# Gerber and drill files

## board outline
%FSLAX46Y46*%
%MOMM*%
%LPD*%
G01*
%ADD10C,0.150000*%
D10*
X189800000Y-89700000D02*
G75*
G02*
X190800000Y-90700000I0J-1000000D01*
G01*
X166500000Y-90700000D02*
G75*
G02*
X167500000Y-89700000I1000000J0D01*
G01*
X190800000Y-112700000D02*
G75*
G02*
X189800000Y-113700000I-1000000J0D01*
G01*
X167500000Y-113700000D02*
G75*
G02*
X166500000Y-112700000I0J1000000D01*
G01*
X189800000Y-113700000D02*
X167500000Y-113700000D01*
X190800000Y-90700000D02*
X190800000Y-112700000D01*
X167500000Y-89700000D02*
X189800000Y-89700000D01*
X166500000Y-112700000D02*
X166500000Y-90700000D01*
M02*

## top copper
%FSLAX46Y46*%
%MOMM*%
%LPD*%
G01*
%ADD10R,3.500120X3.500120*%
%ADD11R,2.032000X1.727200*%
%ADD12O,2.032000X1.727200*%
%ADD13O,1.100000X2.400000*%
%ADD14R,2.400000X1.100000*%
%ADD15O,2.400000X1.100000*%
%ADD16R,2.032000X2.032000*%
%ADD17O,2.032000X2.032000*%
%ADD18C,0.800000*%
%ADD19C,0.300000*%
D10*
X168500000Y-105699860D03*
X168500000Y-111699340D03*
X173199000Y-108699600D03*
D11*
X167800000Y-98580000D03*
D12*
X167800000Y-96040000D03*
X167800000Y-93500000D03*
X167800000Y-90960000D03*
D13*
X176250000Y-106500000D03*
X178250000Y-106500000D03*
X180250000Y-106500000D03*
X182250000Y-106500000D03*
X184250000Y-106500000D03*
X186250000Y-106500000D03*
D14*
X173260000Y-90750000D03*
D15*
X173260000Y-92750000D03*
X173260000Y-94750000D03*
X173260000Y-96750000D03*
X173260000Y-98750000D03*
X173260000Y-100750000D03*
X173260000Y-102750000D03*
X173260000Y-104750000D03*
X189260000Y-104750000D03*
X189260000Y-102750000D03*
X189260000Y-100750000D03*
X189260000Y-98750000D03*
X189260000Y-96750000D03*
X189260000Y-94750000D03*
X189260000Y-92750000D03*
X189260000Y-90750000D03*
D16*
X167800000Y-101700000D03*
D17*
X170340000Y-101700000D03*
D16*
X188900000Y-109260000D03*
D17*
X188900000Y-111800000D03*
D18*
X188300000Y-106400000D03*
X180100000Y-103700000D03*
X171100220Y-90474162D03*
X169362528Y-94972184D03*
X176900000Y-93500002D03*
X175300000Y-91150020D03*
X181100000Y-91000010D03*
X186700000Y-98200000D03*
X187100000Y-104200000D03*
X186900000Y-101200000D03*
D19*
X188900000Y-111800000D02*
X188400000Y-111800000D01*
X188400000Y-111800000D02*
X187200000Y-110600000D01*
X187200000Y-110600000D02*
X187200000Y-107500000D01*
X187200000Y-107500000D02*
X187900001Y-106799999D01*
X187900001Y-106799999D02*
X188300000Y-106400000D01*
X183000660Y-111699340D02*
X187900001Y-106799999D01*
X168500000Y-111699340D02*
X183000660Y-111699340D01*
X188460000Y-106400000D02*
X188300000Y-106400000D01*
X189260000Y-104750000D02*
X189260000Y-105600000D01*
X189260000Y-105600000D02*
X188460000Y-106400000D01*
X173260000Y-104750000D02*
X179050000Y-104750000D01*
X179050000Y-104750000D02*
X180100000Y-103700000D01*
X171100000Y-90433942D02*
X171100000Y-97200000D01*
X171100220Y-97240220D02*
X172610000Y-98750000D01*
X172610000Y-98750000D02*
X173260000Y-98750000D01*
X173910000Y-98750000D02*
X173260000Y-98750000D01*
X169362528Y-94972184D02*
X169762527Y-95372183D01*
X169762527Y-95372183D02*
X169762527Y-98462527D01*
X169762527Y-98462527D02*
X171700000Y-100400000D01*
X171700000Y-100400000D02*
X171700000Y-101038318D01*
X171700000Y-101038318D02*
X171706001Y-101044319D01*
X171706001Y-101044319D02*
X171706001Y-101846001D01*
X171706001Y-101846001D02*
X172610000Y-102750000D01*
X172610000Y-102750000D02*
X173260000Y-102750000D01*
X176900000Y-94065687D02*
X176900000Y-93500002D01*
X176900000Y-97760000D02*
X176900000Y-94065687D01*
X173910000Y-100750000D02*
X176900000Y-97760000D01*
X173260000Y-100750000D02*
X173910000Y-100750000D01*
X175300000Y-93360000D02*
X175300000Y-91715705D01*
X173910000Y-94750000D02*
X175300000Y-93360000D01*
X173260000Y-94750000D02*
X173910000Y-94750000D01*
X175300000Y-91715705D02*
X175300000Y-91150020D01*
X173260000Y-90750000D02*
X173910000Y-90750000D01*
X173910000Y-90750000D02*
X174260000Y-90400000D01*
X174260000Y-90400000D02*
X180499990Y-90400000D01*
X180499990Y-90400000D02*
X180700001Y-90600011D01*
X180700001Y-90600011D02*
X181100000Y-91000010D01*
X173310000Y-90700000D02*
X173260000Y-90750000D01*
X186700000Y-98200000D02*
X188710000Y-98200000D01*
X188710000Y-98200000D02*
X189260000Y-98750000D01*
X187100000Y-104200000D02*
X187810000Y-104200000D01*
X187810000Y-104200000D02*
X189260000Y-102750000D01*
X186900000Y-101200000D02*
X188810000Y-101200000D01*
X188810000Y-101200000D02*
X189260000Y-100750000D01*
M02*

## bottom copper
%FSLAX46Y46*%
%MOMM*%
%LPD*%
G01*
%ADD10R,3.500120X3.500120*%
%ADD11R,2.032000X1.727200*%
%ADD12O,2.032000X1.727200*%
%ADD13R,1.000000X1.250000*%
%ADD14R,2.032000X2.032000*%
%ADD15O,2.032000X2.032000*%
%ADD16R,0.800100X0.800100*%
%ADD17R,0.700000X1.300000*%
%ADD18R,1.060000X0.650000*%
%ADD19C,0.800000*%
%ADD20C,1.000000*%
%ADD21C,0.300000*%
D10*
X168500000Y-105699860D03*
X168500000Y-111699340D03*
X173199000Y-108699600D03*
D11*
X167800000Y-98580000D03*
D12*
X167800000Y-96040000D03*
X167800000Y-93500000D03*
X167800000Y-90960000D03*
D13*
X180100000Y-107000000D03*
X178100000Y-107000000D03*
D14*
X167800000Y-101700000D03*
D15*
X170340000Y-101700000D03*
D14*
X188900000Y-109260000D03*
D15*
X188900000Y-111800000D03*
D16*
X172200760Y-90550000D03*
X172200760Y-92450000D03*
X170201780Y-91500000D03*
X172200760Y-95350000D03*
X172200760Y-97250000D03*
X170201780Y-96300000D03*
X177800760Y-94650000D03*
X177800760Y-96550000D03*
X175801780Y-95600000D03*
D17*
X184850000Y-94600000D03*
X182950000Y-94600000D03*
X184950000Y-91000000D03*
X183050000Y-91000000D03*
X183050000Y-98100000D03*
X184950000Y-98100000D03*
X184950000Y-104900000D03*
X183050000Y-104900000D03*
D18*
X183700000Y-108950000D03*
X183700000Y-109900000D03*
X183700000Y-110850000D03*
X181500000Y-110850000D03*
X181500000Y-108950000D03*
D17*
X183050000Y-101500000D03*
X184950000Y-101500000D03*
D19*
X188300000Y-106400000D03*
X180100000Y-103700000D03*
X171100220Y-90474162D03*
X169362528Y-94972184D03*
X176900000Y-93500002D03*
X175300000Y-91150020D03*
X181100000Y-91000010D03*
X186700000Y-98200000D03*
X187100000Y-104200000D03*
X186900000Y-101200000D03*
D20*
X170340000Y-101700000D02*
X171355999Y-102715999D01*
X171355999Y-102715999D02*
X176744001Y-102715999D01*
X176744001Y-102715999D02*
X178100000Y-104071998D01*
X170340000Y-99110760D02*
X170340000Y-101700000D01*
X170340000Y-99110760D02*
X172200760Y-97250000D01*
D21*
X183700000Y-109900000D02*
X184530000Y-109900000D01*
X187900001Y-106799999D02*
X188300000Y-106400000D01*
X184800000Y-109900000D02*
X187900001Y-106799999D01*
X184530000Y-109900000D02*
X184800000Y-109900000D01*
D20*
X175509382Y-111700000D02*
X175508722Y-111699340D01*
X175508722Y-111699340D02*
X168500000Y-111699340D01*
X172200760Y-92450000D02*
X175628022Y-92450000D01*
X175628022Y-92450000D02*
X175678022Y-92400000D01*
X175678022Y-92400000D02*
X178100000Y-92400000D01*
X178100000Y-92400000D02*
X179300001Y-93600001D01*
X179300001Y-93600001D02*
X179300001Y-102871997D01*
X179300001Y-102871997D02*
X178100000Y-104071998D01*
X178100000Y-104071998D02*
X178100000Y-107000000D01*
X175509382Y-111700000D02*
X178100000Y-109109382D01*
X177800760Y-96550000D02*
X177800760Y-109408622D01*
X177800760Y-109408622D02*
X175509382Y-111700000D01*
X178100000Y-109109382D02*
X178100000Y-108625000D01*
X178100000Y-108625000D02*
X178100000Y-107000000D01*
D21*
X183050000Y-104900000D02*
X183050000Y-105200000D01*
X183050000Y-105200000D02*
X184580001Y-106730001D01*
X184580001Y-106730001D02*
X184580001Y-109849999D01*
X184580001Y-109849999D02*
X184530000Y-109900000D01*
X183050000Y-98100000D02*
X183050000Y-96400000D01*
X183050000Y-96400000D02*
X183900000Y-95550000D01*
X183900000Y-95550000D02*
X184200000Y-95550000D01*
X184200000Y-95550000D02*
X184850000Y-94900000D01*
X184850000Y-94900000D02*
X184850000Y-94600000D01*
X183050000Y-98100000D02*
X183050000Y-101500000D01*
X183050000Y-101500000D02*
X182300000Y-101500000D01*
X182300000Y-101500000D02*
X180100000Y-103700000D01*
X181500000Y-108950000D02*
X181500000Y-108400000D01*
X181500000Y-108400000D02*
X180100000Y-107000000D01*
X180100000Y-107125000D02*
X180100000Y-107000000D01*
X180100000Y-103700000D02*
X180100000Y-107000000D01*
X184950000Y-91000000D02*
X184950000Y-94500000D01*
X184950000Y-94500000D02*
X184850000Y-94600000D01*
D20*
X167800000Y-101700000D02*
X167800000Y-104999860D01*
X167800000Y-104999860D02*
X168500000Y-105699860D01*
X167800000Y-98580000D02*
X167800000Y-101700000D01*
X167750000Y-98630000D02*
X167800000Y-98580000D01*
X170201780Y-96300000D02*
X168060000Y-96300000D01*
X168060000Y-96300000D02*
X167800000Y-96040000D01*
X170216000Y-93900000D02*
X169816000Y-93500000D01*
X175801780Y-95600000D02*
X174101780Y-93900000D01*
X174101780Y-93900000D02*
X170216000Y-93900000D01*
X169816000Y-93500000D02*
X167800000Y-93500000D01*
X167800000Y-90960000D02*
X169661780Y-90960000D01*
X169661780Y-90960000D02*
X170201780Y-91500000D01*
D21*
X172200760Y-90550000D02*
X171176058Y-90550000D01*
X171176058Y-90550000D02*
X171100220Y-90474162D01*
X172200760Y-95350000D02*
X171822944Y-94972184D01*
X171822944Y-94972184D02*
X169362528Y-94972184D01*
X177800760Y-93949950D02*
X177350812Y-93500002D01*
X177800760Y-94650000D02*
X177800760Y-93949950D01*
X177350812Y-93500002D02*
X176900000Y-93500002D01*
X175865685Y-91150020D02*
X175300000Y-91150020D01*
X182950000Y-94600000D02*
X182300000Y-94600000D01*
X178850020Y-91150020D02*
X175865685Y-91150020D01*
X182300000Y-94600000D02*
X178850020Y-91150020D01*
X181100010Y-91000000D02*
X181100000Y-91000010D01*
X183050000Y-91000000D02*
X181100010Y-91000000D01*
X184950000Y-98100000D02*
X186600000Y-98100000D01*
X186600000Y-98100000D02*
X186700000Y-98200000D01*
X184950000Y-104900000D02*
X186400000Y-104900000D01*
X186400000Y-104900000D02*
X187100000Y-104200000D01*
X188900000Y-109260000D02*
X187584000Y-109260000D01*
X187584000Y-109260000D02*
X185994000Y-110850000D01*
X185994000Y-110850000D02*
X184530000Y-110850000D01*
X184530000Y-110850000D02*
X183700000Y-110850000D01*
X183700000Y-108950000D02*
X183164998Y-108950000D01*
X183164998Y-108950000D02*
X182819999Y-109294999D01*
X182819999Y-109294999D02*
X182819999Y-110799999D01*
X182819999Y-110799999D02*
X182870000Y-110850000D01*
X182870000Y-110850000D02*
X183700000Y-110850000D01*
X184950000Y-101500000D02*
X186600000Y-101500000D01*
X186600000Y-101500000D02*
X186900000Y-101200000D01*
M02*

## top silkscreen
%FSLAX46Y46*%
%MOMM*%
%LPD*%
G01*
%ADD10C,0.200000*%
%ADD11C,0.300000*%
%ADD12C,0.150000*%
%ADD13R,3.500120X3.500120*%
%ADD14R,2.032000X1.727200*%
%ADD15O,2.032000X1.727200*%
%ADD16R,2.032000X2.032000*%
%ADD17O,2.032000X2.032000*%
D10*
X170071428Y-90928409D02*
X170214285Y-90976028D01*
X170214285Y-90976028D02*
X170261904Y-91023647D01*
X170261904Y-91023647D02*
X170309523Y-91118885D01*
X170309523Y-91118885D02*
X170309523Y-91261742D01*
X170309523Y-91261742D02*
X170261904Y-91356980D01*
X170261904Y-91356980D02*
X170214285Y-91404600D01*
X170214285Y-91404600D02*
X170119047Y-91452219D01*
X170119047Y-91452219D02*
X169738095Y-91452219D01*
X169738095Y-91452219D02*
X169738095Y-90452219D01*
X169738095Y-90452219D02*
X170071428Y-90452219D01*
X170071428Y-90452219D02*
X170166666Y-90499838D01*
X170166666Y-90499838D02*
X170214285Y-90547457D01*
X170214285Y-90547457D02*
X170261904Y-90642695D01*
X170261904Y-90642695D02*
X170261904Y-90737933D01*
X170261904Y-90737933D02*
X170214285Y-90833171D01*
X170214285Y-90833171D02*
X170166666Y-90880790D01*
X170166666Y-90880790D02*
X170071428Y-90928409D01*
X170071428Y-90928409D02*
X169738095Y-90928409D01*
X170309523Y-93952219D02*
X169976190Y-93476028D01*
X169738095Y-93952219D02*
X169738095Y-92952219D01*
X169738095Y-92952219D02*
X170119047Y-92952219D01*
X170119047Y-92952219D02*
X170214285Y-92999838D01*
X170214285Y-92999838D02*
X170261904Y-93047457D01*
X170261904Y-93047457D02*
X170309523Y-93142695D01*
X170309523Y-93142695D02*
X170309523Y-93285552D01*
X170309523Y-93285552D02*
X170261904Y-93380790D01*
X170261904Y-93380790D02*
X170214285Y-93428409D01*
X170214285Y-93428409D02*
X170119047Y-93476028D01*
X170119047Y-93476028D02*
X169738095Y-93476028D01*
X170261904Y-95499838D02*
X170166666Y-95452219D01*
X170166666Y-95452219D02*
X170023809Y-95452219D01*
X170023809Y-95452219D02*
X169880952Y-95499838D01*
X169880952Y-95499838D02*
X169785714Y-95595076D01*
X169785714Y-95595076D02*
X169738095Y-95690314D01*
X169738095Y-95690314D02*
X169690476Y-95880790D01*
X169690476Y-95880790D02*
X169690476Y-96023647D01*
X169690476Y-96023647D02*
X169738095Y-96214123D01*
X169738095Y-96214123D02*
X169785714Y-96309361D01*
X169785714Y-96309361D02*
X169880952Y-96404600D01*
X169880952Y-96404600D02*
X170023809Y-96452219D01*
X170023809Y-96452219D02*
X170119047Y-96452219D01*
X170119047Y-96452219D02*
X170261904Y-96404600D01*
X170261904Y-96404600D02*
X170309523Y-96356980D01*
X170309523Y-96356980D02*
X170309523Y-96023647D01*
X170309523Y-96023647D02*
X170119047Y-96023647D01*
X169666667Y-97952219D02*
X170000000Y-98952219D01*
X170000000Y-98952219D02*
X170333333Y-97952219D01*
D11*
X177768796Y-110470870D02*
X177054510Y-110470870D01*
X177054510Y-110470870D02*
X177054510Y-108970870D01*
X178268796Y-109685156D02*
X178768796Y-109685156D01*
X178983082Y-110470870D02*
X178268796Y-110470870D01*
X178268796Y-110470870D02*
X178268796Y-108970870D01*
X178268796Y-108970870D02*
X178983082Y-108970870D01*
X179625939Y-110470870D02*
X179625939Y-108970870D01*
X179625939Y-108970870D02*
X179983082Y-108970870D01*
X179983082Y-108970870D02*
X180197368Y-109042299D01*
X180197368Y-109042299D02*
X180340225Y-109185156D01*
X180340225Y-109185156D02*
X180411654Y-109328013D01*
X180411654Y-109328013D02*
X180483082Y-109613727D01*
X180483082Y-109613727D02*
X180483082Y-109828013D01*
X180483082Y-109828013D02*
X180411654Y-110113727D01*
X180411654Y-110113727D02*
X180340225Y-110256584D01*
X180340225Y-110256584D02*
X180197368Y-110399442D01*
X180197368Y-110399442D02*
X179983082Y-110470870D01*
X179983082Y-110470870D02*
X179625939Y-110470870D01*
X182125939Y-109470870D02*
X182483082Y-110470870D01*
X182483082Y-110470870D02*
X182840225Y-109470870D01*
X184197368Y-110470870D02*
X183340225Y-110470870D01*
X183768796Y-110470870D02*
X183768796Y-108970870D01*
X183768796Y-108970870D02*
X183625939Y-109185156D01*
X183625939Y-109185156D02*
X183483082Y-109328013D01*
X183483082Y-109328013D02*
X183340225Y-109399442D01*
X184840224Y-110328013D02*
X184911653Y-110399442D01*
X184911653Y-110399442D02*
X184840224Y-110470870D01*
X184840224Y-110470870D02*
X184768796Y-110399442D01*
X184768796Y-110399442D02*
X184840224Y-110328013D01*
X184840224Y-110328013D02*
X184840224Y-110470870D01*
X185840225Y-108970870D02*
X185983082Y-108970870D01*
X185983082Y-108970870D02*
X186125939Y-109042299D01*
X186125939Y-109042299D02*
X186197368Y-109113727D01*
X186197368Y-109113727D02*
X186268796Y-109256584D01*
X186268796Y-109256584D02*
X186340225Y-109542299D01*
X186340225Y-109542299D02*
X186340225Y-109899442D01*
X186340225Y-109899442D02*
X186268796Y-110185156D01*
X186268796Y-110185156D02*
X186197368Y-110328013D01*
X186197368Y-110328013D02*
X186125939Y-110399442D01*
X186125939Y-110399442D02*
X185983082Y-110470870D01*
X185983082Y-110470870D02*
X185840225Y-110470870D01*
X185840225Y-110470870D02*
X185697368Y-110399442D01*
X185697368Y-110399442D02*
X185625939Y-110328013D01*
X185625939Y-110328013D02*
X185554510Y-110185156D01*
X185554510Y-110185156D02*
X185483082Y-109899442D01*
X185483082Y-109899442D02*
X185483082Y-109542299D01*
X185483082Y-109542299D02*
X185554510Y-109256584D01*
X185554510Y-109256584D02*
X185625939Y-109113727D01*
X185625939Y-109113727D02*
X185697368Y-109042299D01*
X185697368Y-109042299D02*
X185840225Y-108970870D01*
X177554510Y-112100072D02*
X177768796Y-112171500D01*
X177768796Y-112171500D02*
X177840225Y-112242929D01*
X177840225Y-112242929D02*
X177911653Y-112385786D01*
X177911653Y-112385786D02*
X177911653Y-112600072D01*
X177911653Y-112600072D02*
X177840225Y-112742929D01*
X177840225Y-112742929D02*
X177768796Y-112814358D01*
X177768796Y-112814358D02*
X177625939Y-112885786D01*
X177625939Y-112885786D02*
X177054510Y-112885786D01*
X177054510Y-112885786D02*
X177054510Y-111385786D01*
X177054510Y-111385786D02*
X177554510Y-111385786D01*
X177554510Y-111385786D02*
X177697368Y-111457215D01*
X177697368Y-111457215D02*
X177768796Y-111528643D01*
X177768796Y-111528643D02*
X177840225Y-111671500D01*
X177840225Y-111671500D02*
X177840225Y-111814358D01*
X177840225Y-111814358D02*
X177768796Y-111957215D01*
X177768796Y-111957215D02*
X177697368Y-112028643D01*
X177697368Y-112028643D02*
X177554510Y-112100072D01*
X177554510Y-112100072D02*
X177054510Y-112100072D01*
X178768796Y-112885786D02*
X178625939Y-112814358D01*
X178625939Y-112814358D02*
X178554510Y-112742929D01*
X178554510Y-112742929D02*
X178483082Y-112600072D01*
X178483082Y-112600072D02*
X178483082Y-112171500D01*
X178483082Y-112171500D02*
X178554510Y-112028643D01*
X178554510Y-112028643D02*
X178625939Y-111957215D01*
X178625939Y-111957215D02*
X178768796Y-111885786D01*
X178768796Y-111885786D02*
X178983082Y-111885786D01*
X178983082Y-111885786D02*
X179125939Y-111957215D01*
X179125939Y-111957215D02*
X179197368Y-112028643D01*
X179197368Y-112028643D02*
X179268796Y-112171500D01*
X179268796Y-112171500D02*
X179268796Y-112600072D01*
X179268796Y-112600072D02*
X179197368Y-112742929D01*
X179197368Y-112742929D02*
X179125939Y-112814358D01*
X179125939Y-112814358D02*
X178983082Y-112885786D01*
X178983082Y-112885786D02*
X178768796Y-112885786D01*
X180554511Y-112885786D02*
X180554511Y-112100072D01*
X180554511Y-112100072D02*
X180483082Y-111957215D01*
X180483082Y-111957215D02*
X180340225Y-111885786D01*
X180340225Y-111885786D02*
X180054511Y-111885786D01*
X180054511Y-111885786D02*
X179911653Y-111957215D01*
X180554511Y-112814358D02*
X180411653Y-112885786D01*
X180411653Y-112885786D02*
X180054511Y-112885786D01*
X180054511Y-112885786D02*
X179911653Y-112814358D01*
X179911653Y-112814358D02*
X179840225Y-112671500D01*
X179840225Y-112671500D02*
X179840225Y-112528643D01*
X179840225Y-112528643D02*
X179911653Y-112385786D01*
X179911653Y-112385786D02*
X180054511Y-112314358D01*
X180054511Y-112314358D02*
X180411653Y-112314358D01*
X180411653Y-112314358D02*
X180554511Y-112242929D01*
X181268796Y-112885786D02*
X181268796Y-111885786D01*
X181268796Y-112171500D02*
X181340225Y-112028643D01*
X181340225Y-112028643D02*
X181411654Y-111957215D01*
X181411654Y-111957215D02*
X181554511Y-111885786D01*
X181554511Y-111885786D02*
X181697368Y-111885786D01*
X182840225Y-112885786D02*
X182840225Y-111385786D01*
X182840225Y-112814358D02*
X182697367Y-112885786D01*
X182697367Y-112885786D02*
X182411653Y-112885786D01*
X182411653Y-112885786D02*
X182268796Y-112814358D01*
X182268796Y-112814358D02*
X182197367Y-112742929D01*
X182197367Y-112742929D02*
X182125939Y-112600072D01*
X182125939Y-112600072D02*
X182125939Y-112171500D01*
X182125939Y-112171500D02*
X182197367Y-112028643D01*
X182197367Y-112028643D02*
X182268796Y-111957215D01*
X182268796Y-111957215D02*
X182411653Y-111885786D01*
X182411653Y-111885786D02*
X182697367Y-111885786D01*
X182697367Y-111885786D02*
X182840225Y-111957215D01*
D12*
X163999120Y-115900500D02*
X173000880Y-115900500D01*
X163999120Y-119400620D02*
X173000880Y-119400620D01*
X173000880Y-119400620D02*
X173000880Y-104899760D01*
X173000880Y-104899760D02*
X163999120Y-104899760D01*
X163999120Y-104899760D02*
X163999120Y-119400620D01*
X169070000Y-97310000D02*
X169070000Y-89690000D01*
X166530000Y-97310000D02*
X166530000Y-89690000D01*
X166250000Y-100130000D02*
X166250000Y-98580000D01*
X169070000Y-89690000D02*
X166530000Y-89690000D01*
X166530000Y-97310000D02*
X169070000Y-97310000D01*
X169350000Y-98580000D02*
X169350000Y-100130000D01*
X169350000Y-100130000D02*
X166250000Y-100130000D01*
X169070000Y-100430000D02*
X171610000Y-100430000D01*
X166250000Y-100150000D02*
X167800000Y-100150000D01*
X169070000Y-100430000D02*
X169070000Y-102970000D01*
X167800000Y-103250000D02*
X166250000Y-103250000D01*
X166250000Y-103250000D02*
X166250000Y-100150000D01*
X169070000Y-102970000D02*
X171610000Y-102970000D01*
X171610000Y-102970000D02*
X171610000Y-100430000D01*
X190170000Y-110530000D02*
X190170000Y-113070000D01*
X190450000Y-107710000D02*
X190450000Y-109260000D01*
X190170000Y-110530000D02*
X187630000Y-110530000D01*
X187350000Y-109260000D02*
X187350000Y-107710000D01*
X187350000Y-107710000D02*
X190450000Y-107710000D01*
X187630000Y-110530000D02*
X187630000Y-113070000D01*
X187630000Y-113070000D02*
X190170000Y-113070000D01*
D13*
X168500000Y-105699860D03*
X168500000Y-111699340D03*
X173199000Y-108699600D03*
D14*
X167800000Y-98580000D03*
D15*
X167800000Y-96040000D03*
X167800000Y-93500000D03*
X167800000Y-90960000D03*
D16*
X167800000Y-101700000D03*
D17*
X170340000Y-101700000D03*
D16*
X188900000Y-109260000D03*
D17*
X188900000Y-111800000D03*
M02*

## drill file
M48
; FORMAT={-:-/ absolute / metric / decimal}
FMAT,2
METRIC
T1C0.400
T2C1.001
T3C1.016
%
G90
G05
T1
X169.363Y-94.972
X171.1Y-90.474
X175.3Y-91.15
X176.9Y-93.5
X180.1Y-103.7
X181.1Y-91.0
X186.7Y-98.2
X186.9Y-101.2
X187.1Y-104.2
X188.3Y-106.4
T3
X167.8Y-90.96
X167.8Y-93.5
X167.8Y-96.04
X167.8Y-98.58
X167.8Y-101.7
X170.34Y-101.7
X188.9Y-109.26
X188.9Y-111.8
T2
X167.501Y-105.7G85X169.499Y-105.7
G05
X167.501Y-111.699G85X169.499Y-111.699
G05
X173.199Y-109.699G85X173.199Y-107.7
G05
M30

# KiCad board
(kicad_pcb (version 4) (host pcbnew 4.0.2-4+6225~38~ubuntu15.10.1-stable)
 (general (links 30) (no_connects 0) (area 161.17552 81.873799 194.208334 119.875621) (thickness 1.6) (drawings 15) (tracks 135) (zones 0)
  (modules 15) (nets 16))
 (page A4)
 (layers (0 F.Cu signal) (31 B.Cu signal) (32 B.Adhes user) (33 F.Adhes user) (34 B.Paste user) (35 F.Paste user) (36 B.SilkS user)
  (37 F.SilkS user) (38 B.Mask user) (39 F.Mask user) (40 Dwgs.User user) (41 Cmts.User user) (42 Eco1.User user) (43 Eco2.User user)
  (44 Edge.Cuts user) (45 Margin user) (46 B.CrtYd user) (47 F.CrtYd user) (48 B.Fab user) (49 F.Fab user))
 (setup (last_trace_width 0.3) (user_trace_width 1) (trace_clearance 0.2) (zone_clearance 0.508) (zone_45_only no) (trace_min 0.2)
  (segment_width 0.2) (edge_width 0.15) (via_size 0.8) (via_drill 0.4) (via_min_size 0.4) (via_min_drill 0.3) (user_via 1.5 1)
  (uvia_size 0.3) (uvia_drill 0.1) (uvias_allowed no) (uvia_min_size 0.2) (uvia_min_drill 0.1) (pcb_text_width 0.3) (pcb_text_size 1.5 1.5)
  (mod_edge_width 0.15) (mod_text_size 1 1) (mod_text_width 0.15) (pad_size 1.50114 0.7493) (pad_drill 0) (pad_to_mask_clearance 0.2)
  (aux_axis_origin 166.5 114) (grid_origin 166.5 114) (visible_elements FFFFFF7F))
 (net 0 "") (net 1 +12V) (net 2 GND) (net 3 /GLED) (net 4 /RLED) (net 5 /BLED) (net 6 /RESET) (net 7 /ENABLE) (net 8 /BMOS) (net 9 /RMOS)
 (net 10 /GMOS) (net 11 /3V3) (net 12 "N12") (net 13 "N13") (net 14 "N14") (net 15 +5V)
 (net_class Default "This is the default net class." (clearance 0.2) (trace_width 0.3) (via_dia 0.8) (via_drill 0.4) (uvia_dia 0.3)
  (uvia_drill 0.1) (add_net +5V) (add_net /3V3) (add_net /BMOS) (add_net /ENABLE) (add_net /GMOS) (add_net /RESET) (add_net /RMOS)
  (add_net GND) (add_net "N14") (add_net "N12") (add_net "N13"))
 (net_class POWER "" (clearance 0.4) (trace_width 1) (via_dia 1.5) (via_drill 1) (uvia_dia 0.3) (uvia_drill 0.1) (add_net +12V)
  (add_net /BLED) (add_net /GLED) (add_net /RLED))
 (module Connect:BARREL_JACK (layer F.Cu) (at 168.5 111.9 90)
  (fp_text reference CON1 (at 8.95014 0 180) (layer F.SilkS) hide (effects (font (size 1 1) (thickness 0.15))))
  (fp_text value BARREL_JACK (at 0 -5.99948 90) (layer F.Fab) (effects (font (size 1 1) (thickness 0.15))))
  (fp_line (start -4.0005 -4.50088) (end -4.0005 4.50088) (layer F.SilkS) (width 0.15))
  (fp_line (start -7.50062 -4.50088) (end -7.50062 4.50088) (layer F.SilkS) (width 0.15))
  (fp_line (start -7.50062 4.50088) (end 7.00024 4.50088) (layer F.SilkS) (width 0.15))
  (fp_line (start 7.00024 4.50088) (end 7.00024 -4.50088) (layer F.SilkS) (width 0.15))
  (fp_line (start 7.00024 -4.50088) (end -7.50062 -4.50088) (layer F.SilkS) (width 0.15))
  (pad 1 thru_hole rect (at 6.20014 0 90) (size 3.50012 3.50012) (drill oval 1.00076 2.99974) (layers *.Cu *.Mask F.SilkS) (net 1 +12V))
  (pad 2 thru_hole rect (at 0.20066 0 90) (size 3.50012 3.50012) (drill oval 1.00076 2.99974) (layers *.Cu *.Mask F.SilkS) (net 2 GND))
  (pad 3 thru_hole rect (at 3.2004 4.699 90) (size 3.50012 3.50012) (drill oval 2.99974 1.00076) (layers *.Cu *.Mask F.SilkS)))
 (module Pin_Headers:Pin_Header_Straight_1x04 (layer F.Cu) (at 167.8 98.58 180)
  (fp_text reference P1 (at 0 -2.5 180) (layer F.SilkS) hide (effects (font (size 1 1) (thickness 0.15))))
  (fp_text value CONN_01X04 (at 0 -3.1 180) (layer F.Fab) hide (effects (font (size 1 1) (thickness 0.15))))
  (fp_line (start -1.27 1.27) (end -1.27 8.89) (layer F.SilkS) (width 0.15))
  (fp_line (start 1.27 1.27) (end 1.27 8.89) (layer F.SilkS) (width 0.15))
  (fp_line (start 1.55 -1.55) (end 1.55 0) (layer F.SilkS) (width 0.15))
  (fp_line (start -1.27 8.89) (end 1.27 8.89) (layer F.SilkS) (width 0.15))
  (fp_line (start 1.27 1.27) (end -1.27 1.27) (layer F.SilkS) (width 0.15))
  (fp_line (start -1.55 0) (end -1.55 -1.55) (layer F.SilkS) (width 0.15))
  (fp_line (start -1.55 -1.55) (end 1.55 -1.55) (layer F.SilkS) (width 0.15))
  (pad 1 thru_hole rect (at 0 0 180) (size 2.032 1.7272) (drill 1.016) (layers *.Cu *.Mask F.SilkS) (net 1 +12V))
  (pad 2 thru_hole oval (at 0 2.54 180) (size 2.032 1.7272) (drill 1.016) (layers *.Cu *.Mask F.SilkS) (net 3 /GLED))
  (pad 3 thru_hole oval (at 0 5.08 180) (size 2.032 1.7272) (drill 1.016) (layers *.Cu *.Mask F.SilkS) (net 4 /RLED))
  (pad 4 thru_hole oval (at 0 7.62 180) (size 2.032 1.7272) (drill 1.016) (layers *.Cu *.Mask F.SilkS) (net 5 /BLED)))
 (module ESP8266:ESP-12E (layer F.Cu) (at 173.26 90.75)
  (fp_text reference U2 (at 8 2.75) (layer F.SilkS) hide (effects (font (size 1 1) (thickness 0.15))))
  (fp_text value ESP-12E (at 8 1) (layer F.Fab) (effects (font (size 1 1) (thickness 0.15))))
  (pad 9 smd oval (at 2.99 15.75 90) (size 2.4 1.1) (layers F.Cu F.Paste F.Mask))
  (pad 10 smd oval (at 4.99 15.75 90) (size 2.4 1.1) (layers F.Cu F.Paste F.Mask))
  (pad 11 smd oval (at 6.99 15.75 90) (size 2.4 1.1) (layers F.Cu F.Paste F.Mask))
  (pad 12 smd oval (at 8.99 15.75 90) (size 2.4 1.1) (layers F.Cu F.Paste F.Mask))
  (pad 13 smd oval (at 10.99 15.75 90) (size 2.4 1.1) (layers F.Cu F.Paste F.Mask))
  (pad 14 smd oval (at 12.99 15.75 90) (size 2.4 1.1) (layers F.Cu F.Paste F.Mask))
  (pad 1 smd rect (at 0 0) (size 2.4 1.1) (layers F.Cu F.Paste F.Mask) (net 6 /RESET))
  (pad 2 smd oval (at 0 2) (size 2.4 1.1) (layers F.Cu F.Paste F.Mask))
  (pad 3 smd oval (at 0 4) (size 2.4 1.1) (layers F.Cu F.Paste F.Mask) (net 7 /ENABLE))
  (pad 4 smd oval (at 0 6) (size 2.4 1.1) (layers F.Cu F.Paste F.Mask))
  (pad 5 smd oval (at 0 8) (size 2.4 1.1) (layers F.Cu F.Paste F.Mask) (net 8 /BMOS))
  (pad 6 smd oval (at 0 10) (size 2.4 1.1) (layers F.Cu F.Paste F.Mask) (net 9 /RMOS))
  (pad 7 smd oval (at 0 12) (size 2.4 1.1) (layers F.Cu F.Paste F.Mask) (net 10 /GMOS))
  (pad 8 smd oval (at 0 14) (size 2.4 1.1) (layers F.Cu F.Paste F.Mask) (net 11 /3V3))
  (pad 15 smd oval (at 16 14) (size 2.4 1.1) (layers F.Cu F.Paste F.Mask) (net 2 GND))
  (pad 16 smd oval (at 16 12) (size 2.4 1.1) (layers F.Cu F.Paste F.Mask) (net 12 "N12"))
  (pad 17 smd oval (at 16 10) (size 2.4 1.1) (layers F.Cu F.Paste F.Mask) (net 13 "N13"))
  (pad 18 smd oval (at 16 8) (size 2.4 1.1) (layers F.Cu F.Paste F.Mask) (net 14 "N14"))
  (pad 19 smd oval (at 16 6) (size 2.4 1.1) (layers F.Cu F.Paste F.Mask))
  (pad 20 smd oval (at 16 4) (size 2.4 1.1) (layers F.Cu F.Paste F.Mask))
  (pad 21 smd oval (at 16 2) (size 2.4 1.1) (layers F.Cu F.Paste F.Mask))
  (pad 22 smd oval (at 16 0) (size 2.4 1.1) (layers F.Cu F.Paste F.Mask)))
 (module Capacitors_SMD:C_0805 (layer B.Cu) (at 179.1 107 180)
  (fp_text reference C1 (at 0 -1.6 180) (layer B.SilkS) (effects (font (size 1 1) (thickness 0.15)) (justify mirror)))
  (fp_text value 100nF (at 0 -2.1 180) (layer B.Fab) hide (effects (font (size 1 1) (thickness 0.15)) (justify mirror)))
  (pad 1 smd rect (at -1 0 180) (size 1 1.25) (layers B.Cu B.Paste B.Mask) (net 11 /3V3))
  (pad 2 smd rect (at 1 0 180) (size 1 1.25) (layers B.Cu B.Paste B.Mask) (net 2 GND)))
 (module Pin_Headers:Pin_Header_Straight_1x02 (layer F.Cu) (at 167.8 101.7 90)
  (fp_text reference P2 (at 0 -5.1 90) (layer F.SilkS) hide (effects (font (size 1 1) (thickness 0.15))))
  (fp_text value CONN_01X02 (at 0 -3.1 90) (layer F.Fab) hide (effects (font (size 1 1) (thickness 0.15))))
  (fp_line (start 1.27 1.27) (end 1.27 3.81) (layer F.SilkS) (width 0.15))
  (fp_line (start 1.55 -1.55) (end 1.55 0) (layer F.SilkS) (width 0.15))
  (fp_line (start 1.27 1.27) (end -1.27 1.27) (layer F.SilkS) (width 0.15))
  (fp_line (start -1.55 0) (end -1.55 -1.55) (layer F.SilkS) (width 0.15))
  (fp_line (start -1.55 -1.55) (end 1.55 -1.55) (layer F.SilkS) (width 0.15))
  (fp_line (start -1.27 1.27) (end -1.27 3.81) (layer F.SilkS) (width 0.15))
  (fp_line (start -1.27 3.81) (end 1.27 3.81) (layer F.SilkS) (width 0.15))
  (pad 1 thru_hole rect (at 0 0 90) (size 2.032 2.032) (drill 1.016) (layers *.Cu *.Mask F.SilkS) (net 1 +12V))
  (pad 2 thru_hole oval (at 0 2.54 90) (size 2.032 2.032) (drill 1.016) (layers *.Cu *.Mask F.SilkS) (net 2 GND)))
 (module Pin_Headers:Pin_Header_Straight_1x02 (layer F.Cu) (at 188.9 109.26)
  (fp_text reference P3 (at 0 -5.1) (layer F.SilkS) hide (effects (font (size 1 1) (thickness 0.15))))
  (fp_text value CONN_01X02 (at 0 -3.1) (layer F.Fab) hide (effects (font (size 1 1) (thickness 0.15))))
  (fp_line (start 1.27 1.27) (end 1.27 3.81) (layer F.SilkS) (width 0.15))
  (fp_line (start 1.55 -1.55) (end 1.55 0) (layer F.SilkS) (width 0.15))
  (fp_line (start 1.27 1.27) (end -1.27 1.27) (layer F.SilkS) (width 0.15))
  (fp_line (start -1.55 0) (end -1.55 -1.55) (layer F.SilkS) (width 0.15))
  (fp_line (start -1.55 -1.55) (end 1.55 -1.55) (layer F.SilkS) (width 0.15))
  (fp_line (start -1.27 1.27) (end -1.27 3.81) (layer F.SilkS) (width 0.15))
  (fp_line (start -1.27 3.81) (end 1.27 3.81) (layer F.SilkS) (width 0.15))
  (pad 1 thru_hole rect (at 0 0) (size 2.032 2.032) (drill 1.016) (layers *.Cu *.Mask F.SilkS) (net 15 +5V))
  (pad 2 thru_hole oval (at 0 2.54) (size 2.032 2.032) (drill 1.016) (layers *.Cu *.Mask F.SilkS) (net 2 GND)))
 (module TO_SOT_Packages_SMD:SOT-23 (layer B.Cu) (at 171.2 91.5 270)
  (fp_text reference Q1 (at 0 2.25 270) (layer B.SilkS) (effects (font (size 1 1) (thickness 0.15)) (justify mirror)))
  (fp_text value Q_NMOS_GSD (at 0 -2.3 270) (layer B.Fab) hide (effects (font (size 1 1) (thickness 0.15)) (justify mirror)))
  (pad 1 smd rect (at -0.95 -1.00076 270) (size 0.8001 0.8001) (layers B.Cu B.Paste B.Mask) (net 8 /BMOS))
  (pad 2 smd rect (at 0.95 -1.00076 270) (size 0.8001 0.8001) (layers B.Cu B.Paste B.Mask) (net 2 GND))
  (pad 3 smd rect (at 0 0.99822 270) (size 0.8001 0.8001) (layers B.Cu B.Paste B.Mask) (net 5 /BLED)))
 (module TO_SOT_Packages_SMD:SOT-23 (layer B.Cu) (at 171.2 96.3 270)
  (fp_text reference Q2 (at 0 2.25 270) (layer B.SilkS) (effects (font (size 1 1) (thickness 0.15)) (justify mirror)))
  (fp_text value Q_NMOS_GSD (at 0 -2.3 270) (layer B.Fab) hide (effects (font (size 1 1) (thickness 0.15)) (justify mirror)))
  (pad 1 smd rect (at -0.95 -1.00076 270) (size 0.8001 0.8001) (layers B.Cu B.Paste B.Mask) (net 10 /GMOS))
  (pad 2 smd rect (at 0.95 -1.00076 270) (size 0.8001 0.8001) (layers B.Cu B.Paste B.Mask) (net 2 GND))
  (pad 3 smd rect (at 0 0.99822 270) (size 0.8001 0.8001) (layers B.Cu B.Paste B.Mask) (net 3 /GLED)))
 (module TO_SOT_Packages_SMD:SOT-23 (layer B.Cu) (at 176.8 95.6 270)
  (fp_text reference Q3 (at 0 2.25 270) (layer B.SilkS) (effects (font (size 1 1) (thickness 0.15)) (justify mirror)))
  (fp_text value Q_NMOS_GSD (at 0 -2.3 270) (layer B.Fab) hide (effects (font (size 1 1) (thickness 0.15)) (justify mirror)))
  (pad 1 smd rect (at -0.95 -1.00076 270) (size 0.8001 0.8001) (layers B.Cu B.Paste B.Mask) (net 9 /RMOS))
  (pad 2 smd rect (at 0.95 -1.00076 270) (size 0.8001 0.8001) (layers B.Cu B.Paste B.Mask) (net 2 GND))
  (pad 3 smd rect (at 0 0.99822 270) (size 0.8001 0.8001) (layers B.Cu B.Paste B.Mask) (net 4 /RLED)))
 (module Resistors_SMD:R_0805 (layer B.Cu) (at 183.9 94.6 180)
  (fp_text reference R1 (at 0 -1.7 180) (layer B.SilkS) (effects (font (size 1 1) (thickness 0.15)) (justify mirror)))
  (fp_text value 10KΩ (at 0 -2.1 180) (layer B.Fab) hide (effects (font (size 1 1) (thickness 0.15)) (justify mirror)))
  (pad 1 smd rect (at -0.95 0 180) (size 0.7 1.3) (layers B.Cu B.Paste B.Mask) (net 11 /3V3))
  (pad 2 smd rect (at 0.95 0 180) (size 0.7 1.3) (layers B.Cu B.Paste B.Mask) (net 7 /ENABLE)))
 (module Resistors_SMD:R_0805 (layer B.Cu) (at 184 91 180)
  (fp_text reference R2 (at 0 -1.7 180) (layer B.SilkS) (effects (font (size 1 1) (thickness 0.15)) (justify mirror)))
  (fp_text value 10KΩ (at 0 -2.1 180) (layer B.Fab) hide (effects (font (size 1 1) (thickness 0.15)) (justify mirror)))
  (pad 1 smd rect (at -0.95 0 180) (size 0.7 1.3) (layers B.Cu B.Paste B.Mask) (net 11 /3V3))
  (pad 2 smd rect (at 0.95 0 180) (size 0.7 1.3) (layers B.Cu B.Paste B.Mask) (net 6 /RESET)))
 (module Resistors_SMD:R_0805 (layer B.Cu) (at 184 98.1)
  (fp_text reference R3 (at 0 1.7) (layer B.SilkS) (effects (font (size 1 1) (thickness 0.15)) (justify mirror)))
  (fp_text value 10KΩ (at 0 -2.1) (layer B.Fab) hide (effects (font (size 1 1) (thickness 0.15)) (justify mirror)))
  (pad 1 smd rect (at -0.95 0) (size 0.7 1.3) (layers B.Cu B.Paste B.Mask) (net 11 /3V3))
  (pad 2 smd rect (at 0.95 0) (size 0.7 1.3) (layers B.Cu B.Paste B.Mask) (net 14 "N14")))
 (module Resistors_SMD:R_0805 (layer B.Cu) (at 184 104.9 180)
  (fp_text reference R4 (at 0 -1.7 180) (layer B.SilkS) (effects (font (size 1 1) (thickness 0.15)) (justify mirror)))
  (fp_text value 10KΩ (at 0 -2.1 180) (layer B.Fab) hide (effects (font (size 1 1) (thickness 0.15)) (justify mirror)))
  (pad 1 smd rect (at -0.95 0 180) (size 0.7 1.3) (layers B.Cu B.Paste B.Mask) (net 12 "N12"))
  (pad 2 smd rect (at 0.95 0 180) (size 0.7 1.3) (layers B.Cu B.Paste B.Mask) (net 2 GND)))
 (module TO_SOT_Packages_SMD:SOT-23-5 (layer B.Cu) (at 182.6 109.9 180)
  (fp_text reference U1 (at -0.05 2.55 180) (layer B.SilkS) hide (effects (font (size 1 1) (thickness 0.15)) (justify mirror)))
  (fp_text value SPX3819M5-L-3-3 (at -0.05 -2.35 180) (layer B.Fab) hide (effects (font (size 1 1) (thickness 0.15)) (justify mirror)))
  (pad 1 smd rect (at -1.1 0.95 180) (size 1.06 0.65) (layers B.Cu B.Paste B.Mask) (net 15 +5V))
  (pad 2 smd rect (at -1.1 0 180) (size 1.06 0.65) (layers B.Cu B.Paste B.Mask) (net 2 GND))
  (pad 3 smd rect (at -1.1 -0.95 180) (size 1.06 0.65) (layers B.Cu B.Paste B.Mask) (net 15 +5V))
  (pad 4 smd rect (at 1.1 -0.95 180) (size 1.06 0.65) (layers B.Cu B.Paste B.Mask))
  (pad 5 smd rect (at 1.1 0.95 180) (size 1.06 0.65) (layers B.Cu B.Paste B.Mask) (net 11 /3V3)))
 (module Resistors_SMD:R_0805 (layer B.Cu) (at 184 101.5)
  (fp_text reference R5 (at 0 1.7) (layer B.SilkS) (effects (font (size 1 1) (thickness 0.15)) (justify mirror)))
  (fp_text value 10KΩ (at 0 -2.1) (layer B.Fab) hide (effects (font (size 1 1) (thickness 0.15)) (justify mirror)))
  (pad 1 smd rect (at -0.95 0) (size 0.7 1.3) (layers B.Cu B.Paste B.Mask) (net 11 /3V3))
  (pad 2 smd rect (at 0.95 0) (size 0.7 1.3) (layers B.Cu B.Paste B.Mask) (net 13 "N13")))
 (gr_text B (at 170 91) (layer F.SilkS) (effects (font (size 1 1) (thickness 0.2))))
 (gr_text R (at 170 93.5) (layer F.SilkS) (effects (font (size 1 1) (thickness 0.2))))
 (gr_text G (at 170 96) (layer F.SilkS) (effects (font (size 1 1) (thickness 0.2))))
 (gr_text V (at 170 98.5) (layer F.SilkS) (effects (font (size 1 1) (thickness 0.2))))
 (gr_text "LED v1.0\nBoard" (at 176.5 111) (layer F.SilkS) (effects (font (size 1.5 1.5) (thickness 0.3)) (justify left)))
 (gr_arc (start 189.8 90.7) (end 189.8 89.7) (angle 90) (layer Edge.Cuts) (width 0.15))
 (gr_arc (start 167.5 90.7) (end 166.5 90.7) (angle 90) (layer Edge.Cuts) (width 0.15))
 (gr_arc (start 189.8 112.7) (end 190.8 112.7) (angle 90) (layer Edge.Cuts) (width 0.15))
 (gr_arc (start 167.5 112.7) (end 167.5 113.7) (angle 90) (layer Edge.Cuts) (width 0.15))
 (gr_line (start 189.8 113.7) (end 167.5 113.7) (layer Edge.Cuts) (width 0.15))
 (gr_line (start 190.8 90.7) (end 190.8 112.7) (layer Edge.Cuts) (width 0.15))
 (gr_line (start 167.5 89.7) (end 189.8 89.7) (layer Edge.Cuts) (width 0.15))
 (gr_line (start 166.5 112.7) (end 166.5 90.7) (layer Edge.Cuts) (width 0.15))
 (segment (start 170.34 101.7) (end 171.355999 102.715999) (width 1) (layer B.Cu) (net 2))
 (segment (start 171.355999 102.715999) (end 176.744001 102.715999) (width 1) (layer B.Cu) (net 2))
 (segment (start 176.744001 102.715999) (end 178.1 104.071998) (width 1) (layer B.Cu) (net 2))
 (segment (start 170.34 99.11076) (end 170.34 101.7) (width 1) (layer B.Cu) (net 2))
 (segment (start 170.34 99.11076) (end 172.20076 97.25) (width 1) (layer B.Cu) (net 2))
 (segment (start 188.9 111.8) (end 188.4 111.8) (width 0.3) (layer F.Cu) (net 2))
 (segment (start 188.4 111.8) (end 187.2 110.6) (width 0.3) (layer F.Cu) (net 2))
 (segment (start 187.2 110.6) (end 187.2 107.5) (width 0.3) (layer F.Cu) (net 2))
 (segment (start 187.2 107.5) (end 187.900001 106.799999) (width 0.3) (layer F.Cu) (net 2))
 (segment (start 187.900001 106.799999) (end 188.3 106.4) (width 0.3) (layer F.Cu) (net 2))
 (segment (start 183.7 109.9) (end 184.53 109.9) (width 0.3) (layer B.Cu) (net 2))
 (segment (start 183.00066 111.69934) (end 187.900001 106.799999) (width 0.3) (layer F.Cu) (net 2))
 (segment (start 168.5 111.69934) (end 183.00066 111.69934) (width 0.3) (layer F.Cu) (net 2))
 (segment (start 187.900001 106.799999) (end 188.3 106.4) (width 0.3) (layer B.Cu) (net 2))
 (segment (start 184.8 109.9) (end 187.900001 106.799999) (width 0.3) (layer B.Cu) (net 2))
 (segment (start 188.46 106.4) (end 188.3 106.4) (width 0.3) (layer F.Cu) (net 2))
 (segment (start 189.26 104.75) (end 189.26 105.6) (width 0.3) (layer F.Cu) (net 2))
 (segment (start 189.26 105.6) (end 188.46 106.4) (width 0.3) (layer F.Cu) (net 2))
 (segment (start 184.53 109.9) (end 184.8 109.9) (width 0.3) (layer B.Cu) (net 2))
 (segment (start 175.509382 111.7) (end 175.508722 111.69934) (width 1) (layer B.Cu) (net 2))
 (segment (start 175.508722 111.69934) (end 168.5 111.69934) (width 1) (layer B.Cu) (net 2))
 (segment (start 172.20076 92.45) (end 175.628022 92.45) (width 1) (layer B.Cu) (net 2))
 (segment (start 175.628022 92.45) (end 175.678022 92.4) (width 1) (layer B.Cu) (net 2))
 (segment (start 175.678022 92.4) (end 178.1 92.4) (width 1) (layer B.Cu) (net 2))
 (segment (start 178.1 92.4) (end 179.300001 93.600001) (width 1) (layer B.Cu) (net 2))
 (segment (start 179.300001 93.600001) (end 179.300001 102.871997) (width 1) (layer B.Cu) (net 2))
 (segment (start 179.300001 102.871997) (end 178.1 104.071998) (width 1) (layer B.Cu) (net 2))
 (segment (start 178.1 104.071998) (end 178.1 107) (width 1) (layer B.Cu) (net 2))
 (segment (start 175.509382 111.7) (end 178.1 109.109382) (width 1) (layer B.Cu) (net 2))
 (segment (start 177.80076 96.55) (end 177.80076 109.408622) (width 1) (layer B.Cu) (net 2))
 (segment (start 177.80076 109.408622) (end 175.509382 111.7) (width 1) (layer B.Cu) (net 2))
 (segment (start 178.1 109.109382) (end 178.1 108.625) (width 1) (layer B.Cu) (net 2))
 (segment (start 178.1 108.625) (end 178.1 107) (width 1) (layer B.Cu) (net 2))
 (segment (start 183.05 104.9) (end 183.05 105.2) (width 0.3) (layer B.Cu) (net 2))
 (segment (start 183.05 105.2) (end 184.580001 106.730001) (width 0.3) (layer B.Cu) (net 2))
 (segment (start 184.580001 106.730001) (end 184.580001 109.849999) (width 0.3) (layer B.Cu) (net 2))
 (segment (start 184.580001 109.849999) (end 184.53 109.9) (width 0.3) (layer B.Cu) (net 2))
 (segment (start 183.05 98.1) (end 183.05 96.4) (width 0.3) (layer B.Cu) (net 11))
 (segment (start 183.05 96.4) (end 183.9 95.55) (width 0.3) (layer B.Cu) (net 11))
 (segment (start 183.9 95.55) (end 184.2 95.55) (width 0.3) (layer B.Cu) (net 11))
 (segment (start 184.2 95.55) (end 184.85 94.9) (width 0.3) (layer B.Cu) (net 11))
 (segment (start 184.85 94.9) (end 184.85 94.6) (width 0.3) (layer B.Cu) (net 11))
 (segment (start 183.05 98.1) (end 183.05 101.5) (width 0.3) (layer B.Cu) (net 11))
 (segment (start 183.05 101.5) (end 182.3 101.5) (width 0.3) (layer B.Cu) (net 11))
 (segment (start 182.3 101.5) (end 180.1 103.7) (width 0.3) (layer B.Cu) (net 11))
 (segment (start 181.5 108.95) (end 181.5 108.4) (width 0.3) (layer B.Cu) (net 11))
 (segment (start 181.5 108.4) (end 180.1 107) (width 0.3) (layer B.Cu) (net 11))
 (segment (start 180.1 107.125) (end 180.1 107) (width 0.3) (layer B.Cu) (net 11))
 (segment (start 173.26 104.75) (end 179.05 104.75) (width 0.3) (layer F.Cu) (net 11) (status 10))
 (segment (start 179.05 104.75) (end 180.1 103.7) (width 0.3) (layer F.Cu) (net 11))
 (segment (start 180.1 103.7) (end 180.1 107) (width 0.3) (layer B.Cu) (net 11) (status 20))
 (segment (start 184.95 91) (end 184.95 94.5) (width 0.3) (layer B.Cu) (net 11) (status 30))
 (segment (start 184.95 94.5) (end 184.85 94.6) (width 0.3) (layer B.Cu) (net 11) (status 30))
 (segment (start 167.8 101.7) (end 167.8 104.99986) (width 1) (layer B.Cu) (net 1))
 (segment (start 167.8 104.99986) (end 168.5 105.69986) (width 1) (layer B.Cu) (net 1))
 (segment (start 167.8 98.58) (end 167.8 101.7) (width 1) (layer B.Cu) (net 1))
 (segment (start 167.75 98.63) (end 167.8 98.58) (width 1) (layer B.Cu) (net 1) (status 30))
 (segment (start 170.20178 96.3) (end 168.06 96.3) (width 1) (layer B.Cu) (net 3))
 (segment (start 168.06 96.3) (end 167.8 96.04) (width 1) (layer B.Cu) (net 3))
 (segment (start 170.216 93.9) (end 169.816 93.5) (width 1) (layer B.Cu) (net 4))
 (segment (start 175.80178 95.6) (end 174.10178 93.9) (width 1) (layer B.Cu) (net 4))
 (segment (start 174.10178 93.9) (end 170.216 93.9) (width 1) (layer B.Cu) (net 4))
 (segment (start 169.816 93.5) (end 167.8 93.5) (width 1) (layer B.Cu) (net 4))
 (segment (start 167.8 90.96) (end 169.66178 90.96) (width 1) (layer B.Cu) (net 5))
 (segment (start 169.66178 90.96) (end 170.20178 91.5) (width 1) (layer B.Cu) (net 5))
 (segment (start 171.1 90.433942) (end 171.1 97.2) (width 0.3) (layer F.Cu) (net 8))
 (segment (start 171.10022 97.24022) (end 172.61 98.75) (width 0.3) (layer F.Cu) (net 8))
 (segment (start 172.61 98.75) (end 173.26 98.75) (width 0.3) (layer F.Cu) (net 8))
 (segment (start 172.20076 90.55) (end 171.176058 90.55) (width 0.3) (layer B.Cu) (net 8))
 (segment (start 171.176058 90.55) (end 171.10022 90.474162) (width 0.3) (layer B.Cu) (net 8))
 (segment (start 173.91 98.75) (end 173.26 98.75) (width 0.3) (layer F.Cu) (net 8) (status 30))
 (segment (start 169.362528 94.972184) (end 169.762527 95.372183) (width 0.3) (layer F.Cu) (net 10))
 (segment (start 169.762527 95.372183) (end 169.762527 98.462527) (width 0.3) (layer F.Cu) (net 10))
 (segment (start 169.762527 98.462527) (end 171.7 100.4) (width 0.3) (layer F.Cu) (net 10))
 (segment (start 171.7 100.4) (end 171.7 101.038318) (width 0.3) (layer F.Cu) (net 10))
 (segment (start 171.7 101.038318) (end 171.706001 101.044319) (width 0.3) (layer F.Cu) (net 10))
 (segment (start 171.706001 101.044319) (end 171.706001 101.846001) (width 0.3) (layer F.Cu) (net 10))
 (segment (start 171.706001 101.846001) (end 172.61 102.75) (width 0.3) (layer F.Cu) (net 10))
 (segment (start 172.61 102.75) (end 173.26 102.75) (width 0.3) (layer F.Cu) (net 10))
 (segment (start 172.20076 95.35) (end 171.822944 94.972184) (width 0.3) (layer B.Cu) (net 10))
 (segment (start 171.822944 94.972184) (end 169.362528 94.972184) (width 0.3) (layer B.Cu) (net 10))
 (segment (start 177.80076 93.94995) (end 177.350812 93.500002) (width 0.3) (layer B.Cu) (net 9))
 (segment (start 176.9 94.065687) (end 176.9 93.500002) (width 0.3) (layer F.Cu) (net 9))
 (segment (start 176.9 97.76) (end 176.9 94.065687) (width 0.3) (layer F.Cu) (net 9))
 (segment (start 173.91 100.75) (end 176.9 97.76) (width 0.3) (layer F.Cu) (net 9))
 (segment (start 177.80076 94.65) (end 177.80076 93.94995) (width 0.3) (layer B.Cu) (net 9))
 (segment (start 173.26 100.75) (end 173.91 100.75) (width 0.3) (layer F.Cu) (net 9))
 (segment (start 177.350812 93.500002) (end 176.9 93.500002) (width 0.3) (layer B.Cu) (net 9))
 (segment (start 175.3 93.36) (end 175.3 91.715705) (width 0.3) (layer F.Cu) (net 7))
 (segment (start 173.91 94.75) (end 175.3 93.36) (width 0.3) (layer F.Cu) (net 7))
 (segment (start 173.26 94.75) (end 173.91 94.75) (width 0.3) (layer F.Cu) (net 7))
 (segment (start 175.865685 91.15002) (end 175.3 91.15002) (width 0.3) (layer B.Cu) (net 7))
 (segment (start 182.95 94.6) (end 182.3 94.6) (width 0.3) (layer B.Cu) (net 7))
 (segment (start 178.85002 91.15002) (end 175.865685 91.15002) (width 0.3) (layer B.Cu) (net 7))
 (segment (start 175.3 91.715705) (end 175.3 91.15002) (width 0.3) (layer F.Cu) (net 7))
 (segment (start 182.3 94.6) (end 178.85002 91.15002) (width 0.3) (layer B.Cu) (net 7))
 (segment (start 173.26 90.75) (end 173.91 90.75) (width 0.3) (layer F.Cu) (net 6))
 (segment (start 173.91 90.75) (end 174.26 90.4) (width 0.3) (layer F.Cu) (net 6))
 (segment (start 174.26 90.4) (end 180.49999 90.4) (width 0.3) (layer F.Cu) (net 6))
 (segment (start 180.49999 90.4) (end 180.700001 90.600011) (width 0.3) (layer F.Cu) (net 6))
 (segment (start 180.700001 90.600011) (end 181.1 91.00001) (width 0.3) (layer F.Cu) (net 6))
 (segment (start 181.10001 91) (end 181.1 91.00001) (width 0.3) (layer B.Cu) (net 6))
 (segment (start 183.05 91) (end 181.10001 91) (width 0.3) (layer B.Cu) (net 6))
 (segment (start 173.31 90.7) (end 173.26 90.75) (width 0.3) (layer F.Cu) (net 6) (status 30))
 (segment (start 186.7 98.2) (end 188.71 98.2) (width 0.3) (layer F.Cu) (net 14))
 (segment (start 188.71 98.2) (end 189.26 98.75) (width 0.3) (layer F.Cu) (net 14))
 (segment (start 184.95 98.1) (end 186.6 98.1) (width 0.3) (layer B.Cu) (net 14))
 (segment (start 186.6 98.1) (end 186.7 98.2) (width 0.3) (layer B.Cu) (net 14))
 (segment (start 187.1 104.2) (end 187.81 104.2) (width 0.3) (layer F.Cu) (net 12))
 (segment (start 187.81 104.2) (end 189.26 102.75) (width 0.3) (layer F.Cu) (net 12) (status 20))
 (segment (start 184.95 104.9) (end 186.4 104.9) (width 0.3) (layer B.Cu) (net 12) (status 10))
 (segment (start 186.4 104.9) (end 187.1 104.2) (width 0.3) (layer B.Cu) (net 12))
 (segment (start 188.9 109.26) (end 187.584 109.26) (width 0.3) (layer B.Cu) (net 15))
 (segment (start 187.584 109.26) (end 185.994 110.85) (width 0.3) (layer B.Cu) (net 15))
 (segment (start 185.994 110.85) (end 184.53 110.85) (width 0.3) (layer B.Cu) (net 15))
 (segment (start 184.53 110.85) (end 183.7 110.85) (width 0.3) (layer B.Cu) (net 15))
 (segment (start 183.7 108.95) (end 183.164998 108.95) (width 0.3) (layer B.Cu) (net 15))
 (segment (start 183.164998 108.95) (end 182.819999 109.294999) (width 0.3) (layer B.Cu) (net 15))
 (segment (start 182.819999 109.294999) (end 182.819999 110.799999) (width 0.3) (layer B.Cu) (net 15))
 (segment (start 182.819999 110.799999) (end 182.87 110.85) (width 0.3) (layer B.Cu) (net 15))
 (segment (start 182.87 110.85) (end 183.7 110.85) (width 0.3) (layer B.Cu) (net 15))
 (segment (start 186.9 101.2) (end 188.81 101.2) (width 0.3) (layer F.Cu) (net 13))
 (segment (start 188.81 101.2) (end 189.26 100.75) (width 0.3) (layer F.Cu) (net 13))
 (segment (start 184.95 101.5) (end 186.6 101.5) (width 0.3) (layer B.Cu) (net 13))
 (segment (start 186.6 101.5) (end 186.9 101.2) (width 0.3) (layer B.Cu) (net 13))
 (via (at 188.3 106.4) (size 0.8) (drill 0.4) (layers F.Cu B.Cu) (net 2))
 (via (at 180.1 103.7) (size 0.8) (drill 0.4) (layers F.Cu B.Cu) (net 11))
 (via (at 171.10022 90.474162) (size 0.8) (drill 0.4) (layers F.Cu B.Cu) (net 8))
 (via (at 169.362528 94.972184) (size 0.8) (drill 0.4) (layers F.Cu B.Cu) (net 10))
 (via (at 176.9 93.500002) (size 0.8) (drill 0.4) (layers F.Cu B.Cu) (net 9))
 (via (at 175.3 91.15002) (size 0.8) (drill 0.4) (layers F.Cu B.Cu) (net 7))
 (via (at 181.1 91.00001) (size 0.8) (drill 0.4) (layers F.Cu B.Cu) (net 6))
 (via (at 186.7 98.2) (size 0.8) (drill 0.4) (layers F.Cu B.Cu) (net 14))
 (via (at 187.1 104.2) (size 0.8) (drill 0.4) (layers F.Cu B.Cu) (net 12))
 (via (at 186.9 101.2) (size 0.8) (drill 0.4) (layers F.Cu B.Cu) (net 13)))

